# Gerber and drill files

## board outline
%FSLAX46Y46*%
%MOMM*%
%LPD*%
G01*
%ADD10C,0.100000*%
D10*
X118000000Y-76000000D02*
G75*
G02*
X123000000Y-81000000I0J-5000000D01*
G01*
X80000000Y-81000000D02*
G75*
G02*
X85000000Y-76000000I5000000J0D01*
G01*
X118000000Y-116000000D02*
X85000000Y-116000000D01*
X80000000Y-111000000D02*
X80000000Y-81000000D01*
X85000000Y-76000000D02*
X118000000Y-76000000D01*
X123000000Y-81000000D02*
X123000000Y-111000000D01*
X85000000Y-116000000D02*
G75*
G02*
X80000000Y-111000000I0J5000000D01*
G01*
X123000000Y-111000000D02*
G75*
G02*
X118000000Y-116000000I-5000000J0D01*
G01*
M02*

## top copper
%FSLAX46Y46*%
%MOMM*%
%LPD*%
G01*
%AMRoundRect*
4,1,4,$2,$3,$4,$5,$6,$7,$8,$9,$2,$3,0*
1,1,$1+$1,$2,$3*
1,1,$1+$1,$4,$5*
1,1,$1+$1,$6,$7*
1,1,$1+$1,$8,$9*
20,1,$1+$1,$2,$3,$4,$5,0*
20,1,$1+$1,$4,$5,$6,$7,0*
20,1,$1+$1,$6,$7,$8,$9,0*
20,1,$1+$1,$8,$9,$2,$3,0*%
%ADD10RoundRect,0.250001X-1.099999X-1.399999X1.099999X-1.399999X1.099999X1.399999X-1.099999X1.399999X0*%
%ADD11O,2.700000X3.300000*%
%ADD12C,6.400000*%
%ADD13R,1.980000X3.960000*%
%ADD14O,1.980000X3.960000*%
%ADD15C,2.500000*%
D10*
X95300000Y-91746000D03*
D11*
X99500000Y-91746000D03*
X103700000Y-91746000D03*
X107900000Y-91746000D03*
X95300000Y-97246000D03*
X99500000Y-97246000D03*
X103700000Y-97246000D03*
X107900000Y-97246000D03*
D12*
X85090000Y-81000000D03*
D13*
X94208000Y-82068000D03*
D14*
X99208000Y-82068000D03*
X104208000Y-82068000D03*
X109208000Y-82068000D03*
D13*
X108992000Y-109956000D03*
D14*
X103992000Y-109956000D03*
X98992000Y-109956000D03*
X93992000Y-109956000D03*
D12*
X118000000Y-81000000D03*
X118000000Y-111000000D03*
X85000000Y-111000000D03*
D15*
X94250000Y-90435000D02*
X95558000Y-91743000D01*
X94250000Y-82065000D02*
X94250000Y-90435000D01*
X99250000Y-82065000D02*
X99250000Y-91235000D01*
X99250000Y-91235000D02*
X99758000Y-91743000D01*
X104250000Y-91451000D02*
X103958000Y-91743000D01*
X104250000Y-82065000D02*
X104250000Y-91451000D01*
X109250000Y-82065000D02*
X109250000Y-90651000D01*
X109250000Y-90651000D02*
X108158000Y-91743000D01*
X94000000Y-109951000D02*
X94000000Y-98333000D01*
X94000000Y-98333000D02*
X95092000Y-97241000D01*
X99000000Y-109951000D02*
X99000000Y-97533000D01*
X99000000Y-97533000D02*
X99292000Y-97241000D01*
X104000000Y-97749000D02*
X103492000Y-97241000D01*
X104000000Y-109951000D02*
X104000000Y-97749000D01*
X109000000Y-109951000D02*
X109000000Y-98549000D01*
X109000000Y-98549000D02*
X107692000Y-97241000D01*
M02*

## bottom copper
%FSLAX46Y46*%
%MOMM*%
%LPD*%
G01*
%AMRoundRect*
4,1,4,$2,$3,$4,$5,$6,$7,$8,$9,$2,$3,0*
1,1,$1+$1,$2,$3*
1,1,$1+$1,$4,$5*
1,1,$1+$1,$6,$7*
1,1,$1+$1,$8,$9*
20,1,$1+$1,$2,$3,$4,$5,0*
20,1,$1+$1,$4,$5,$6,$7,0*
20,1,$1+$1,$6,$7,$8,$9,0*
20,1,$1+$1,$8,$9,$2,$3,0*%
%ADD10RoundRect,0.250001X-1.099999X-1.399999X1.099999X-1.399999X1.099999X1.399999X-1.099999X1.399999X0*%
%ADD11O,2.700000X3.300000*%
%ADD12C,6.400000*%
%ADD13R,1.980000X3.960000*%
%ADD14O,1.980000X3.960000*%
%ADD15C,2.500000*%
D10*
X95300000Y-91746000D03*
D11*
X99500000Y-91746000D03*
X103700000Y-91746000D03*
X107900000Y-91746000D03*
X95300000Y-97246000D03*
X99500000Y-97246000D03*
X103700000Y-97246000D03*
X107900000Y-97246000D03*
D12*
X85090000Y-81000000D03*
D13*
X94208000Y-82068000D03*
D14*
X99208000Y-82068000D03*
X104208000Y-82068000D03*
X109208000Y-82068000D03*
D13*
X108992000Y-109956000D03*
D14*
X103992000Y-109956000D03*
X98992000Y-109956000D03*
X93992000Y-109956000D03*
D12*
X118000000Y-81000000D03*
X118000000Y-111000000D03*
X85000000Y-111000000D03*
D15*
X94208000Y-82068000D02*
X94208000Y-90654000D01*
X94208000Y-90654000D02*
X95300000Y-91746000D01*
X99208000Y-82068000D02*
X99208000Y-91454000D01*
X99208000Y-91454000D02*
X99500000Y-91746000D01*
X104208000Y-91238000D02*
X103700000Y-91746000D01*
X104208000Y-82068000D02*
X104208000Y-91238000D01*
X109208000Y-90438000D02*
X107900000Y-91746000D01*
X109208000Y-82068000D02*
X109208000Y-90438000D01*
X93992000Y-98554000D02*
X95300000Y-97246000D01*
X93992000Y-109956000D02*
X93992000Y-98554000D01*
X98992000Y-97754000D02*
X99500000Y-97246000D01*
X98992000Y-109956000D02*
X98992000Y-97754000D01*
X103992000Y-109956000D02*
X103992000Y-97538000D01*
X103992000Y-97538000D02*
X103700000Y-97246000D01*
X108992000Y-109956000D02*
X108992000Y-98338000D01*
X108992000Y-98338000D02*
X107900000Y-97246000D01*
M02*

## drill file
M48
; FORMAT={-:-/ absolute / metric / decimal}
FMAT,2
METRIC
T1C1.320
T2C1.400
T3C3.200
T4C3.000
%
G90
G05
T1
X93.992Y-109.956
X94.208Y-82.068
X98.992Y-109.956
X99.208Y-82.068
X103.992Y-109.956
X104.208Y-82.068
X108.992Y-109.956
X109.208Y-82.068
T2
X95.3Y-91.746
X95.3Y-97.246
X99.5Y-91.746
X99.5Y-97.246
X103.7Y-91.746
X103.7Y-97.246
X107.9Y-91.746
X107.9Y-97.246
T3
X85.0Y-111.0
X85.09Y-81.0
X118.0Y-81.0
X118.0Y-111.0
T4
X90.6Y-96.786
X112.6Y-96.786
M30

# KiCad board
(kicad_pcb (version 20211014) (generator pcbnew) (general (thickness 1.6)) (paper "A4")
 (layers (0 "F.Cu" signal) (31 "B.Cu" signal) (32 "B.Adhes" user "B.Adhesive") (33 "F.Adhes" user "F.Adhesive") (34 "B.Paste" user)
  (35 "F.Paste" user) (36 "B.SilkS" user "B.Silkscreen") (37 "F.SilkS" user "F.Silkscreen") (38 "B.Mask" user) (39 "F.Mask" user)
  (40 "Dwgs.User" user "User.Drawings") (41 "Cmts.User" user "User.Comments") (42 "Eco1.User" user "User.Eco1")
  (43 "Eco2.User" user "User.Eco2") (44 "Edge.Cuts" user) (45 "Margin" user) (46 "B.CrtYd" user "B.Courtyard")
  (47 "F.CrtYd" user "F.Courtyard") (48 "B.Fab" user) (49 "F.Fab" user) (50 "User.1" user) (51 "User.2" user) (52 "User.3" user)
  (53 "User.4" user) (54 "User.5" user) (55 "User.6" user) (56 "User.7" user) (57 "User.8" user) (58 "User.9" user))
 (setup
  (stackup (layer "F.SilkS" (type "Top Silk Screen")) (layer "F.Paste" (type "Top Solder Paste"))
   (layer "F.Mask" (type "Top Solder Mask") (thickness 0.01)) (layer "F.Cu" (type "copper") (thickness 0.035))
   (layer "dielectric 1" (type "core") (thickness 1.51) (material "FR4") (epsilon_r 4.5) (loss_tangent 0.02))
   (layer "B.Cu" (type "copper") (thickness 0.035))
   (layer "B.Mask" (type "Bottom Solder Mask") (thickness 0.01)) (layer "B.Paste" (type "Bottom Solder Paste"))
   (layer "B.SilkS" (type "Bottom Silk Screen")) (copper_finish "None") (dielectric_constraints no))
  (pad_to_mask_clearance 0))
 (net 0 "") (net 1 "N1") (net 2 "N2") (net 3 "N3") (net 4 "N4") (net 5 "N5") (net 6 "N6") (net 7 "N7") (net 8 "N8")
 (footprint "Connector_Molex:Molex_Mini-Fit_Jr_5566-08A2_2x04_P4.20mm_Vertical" (layer "F.Cu") (at 95.3 91.746)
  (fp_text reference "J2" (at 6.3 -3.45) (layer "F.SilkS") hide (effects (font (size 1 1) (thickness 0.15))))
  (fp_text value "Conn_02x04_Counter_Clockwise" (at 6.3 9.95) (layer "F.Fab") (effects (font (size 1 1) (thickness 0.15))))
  (pad "" np_thru_hole circle (at 17.3 5.04) (size 3 3) (drill 3) (layers *.Cu *.Mask))
  (pad "" np_thru_hole circle (at -4.7 5.04) (size 3 3) (drill 3) (layers *.Cu *.Mask))
  (pad "1" thru_hole roundrect (at 0 0) (size 2.7 3.3) (drill 1.4) (layers *.Cu *.Mask) (roundrect_rratio 0.092593) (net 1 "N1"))
  (pad "2" thru_hole oval (at 4.2 0) (size 2.7 3.3) (drill 1.4) (layers *.Cu *.Mask) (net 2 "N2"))
  (pad "3" thru_hole oval (at 8.4 0) (size 2.7 3.3) (drill 1.4) (layers *.Cu *.Mask) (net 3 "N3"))
  (pad "4" thru_hole oval (at 12.6 0) (size 2.7 3.3) (drill 1.4) (layers *.Cu *.Mask) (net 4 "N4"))
  (pad "5" thru_hole oval (at 0 5.5) (size 2.7 3.3) (drill 1.4) (layers *.Cu *.Mask) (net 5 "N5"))
  (pad "6" thru_hole oval (at 4.2 5.5) (size 2.7 3.3) (drill 1.4) (layers *.Cu *.Mask) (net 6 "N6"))
  (pad "7" thru_hole oval (at 8.4 5.5) (size 2.7 3.3) (drill 1.4) (layers *.Cu *.Mask) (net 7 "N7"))
  (pad "8" thru_hole oval (at 12.6 5.5) (size 2.7 3.3) (drill 1.4) (layers *.Cu *.Mask) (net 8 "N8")))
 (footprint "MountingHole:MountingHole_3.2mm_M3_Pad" (layer "F.Cu") (at 85.09 81)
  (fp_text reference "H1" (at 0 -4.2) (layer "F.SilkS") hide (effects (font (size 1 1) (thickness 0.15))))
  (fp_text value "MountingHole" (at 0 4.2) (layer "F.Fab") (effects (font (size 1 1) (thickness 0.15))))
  (pad "1" thru_hole circle (at 0 0) (size 6.4 6.4) (drill 3.2) (layers *.Cu *.Mask)))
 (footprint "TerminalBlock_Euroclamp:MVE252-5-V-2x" (layer "F.Cu") (at 101.6 82.296)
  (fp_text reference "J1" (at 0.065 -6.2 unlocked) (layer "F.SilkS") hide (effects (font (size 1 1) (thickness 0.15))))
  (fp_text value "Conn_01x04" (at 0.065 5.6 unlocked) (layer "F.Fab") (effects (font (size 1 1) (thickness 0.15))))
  (pad "1" thru_hole rect (at -7.392 -0.228) (size 1.98 3.96) (drill 1.32) (layers *.Cu *.Mask) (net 1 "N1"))
  (pad "2" thru_hole oval (at -2.392 -0.228) (size 1.98 3.96) (drill 1.32) (layers *.Cu *.Mask) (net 2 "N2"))
  (pad "3" thru_hole oval (at 2.608 -0.228) (size 1.98 3.96) (drill 1.32) (layers *.Cu *.Mask) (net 3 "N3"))
  (pad "4" thru_hole oval (at 7.608 -0.228) (size 1.98 3.96) (drill 1.32) (layers *.Cu *.Mask) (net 4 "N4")))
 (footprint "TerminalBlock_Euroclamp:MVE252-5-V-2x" (layer "F.Cu") (at 101.6 109.728 180)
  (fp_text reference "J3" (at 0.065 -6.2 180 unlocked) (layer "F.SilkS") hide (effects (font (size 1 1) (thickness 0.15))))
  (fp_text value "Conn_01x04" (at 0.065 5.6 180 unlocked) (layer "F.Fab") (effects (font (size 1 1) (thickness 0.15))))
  (pad "1" thru_hole rect (at -7.392 -0.228 180) (size 1.98 3.96) (drill 1.32) (layers *.Cu *.Mask) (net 8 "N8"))
  (pad "2" thru_hole oval (at -2.392 -0.228 180) (size 1.98 3.96) (drill 1.32) (layers *.Cu *.Mask) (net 7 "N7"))
  (pad "3" thru_hole oval (at 2.608 -0.228 180) (size 1.98 3.96) (drill 1.32) (layers *.Cu *.Mask) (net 6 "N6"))
  (pad "4" thru_hole oval (at 7.608 -0.228 180) (size 1.98 3.96) (drill 1.32) (layers *.Cu *.Mask) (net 5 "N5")))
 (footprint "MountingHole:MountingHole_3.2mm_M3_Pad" (layer "F.Cu") (at 118 81)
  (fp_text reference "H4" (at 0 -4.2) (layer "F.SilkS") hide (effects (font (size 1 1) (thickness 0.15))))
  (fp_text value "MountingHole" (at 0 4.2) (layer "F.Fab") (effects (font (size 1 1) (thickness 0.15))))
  (pad "1" thru_hole circle (at 0 0) (size 6.4 6.4) (drill 3.2) (layers *.Cu *.Mask)))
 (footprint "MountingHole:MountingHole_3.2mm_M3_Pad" (layer "F.Cu") (at 118 111)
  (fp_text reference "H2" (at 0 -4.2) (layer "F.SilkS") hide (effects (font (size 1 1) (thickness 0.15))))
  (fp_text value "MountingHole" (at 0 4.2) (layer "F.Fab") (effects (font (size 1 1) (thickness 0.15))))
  (pad "1" thru_hole circle (at 0 0) (size 6.4 6.4) (drill 3.2) (layers *.Cu *.Mask)))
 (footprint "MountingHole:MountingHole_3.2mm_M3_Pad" (layer "F.Cu") (at 85 111)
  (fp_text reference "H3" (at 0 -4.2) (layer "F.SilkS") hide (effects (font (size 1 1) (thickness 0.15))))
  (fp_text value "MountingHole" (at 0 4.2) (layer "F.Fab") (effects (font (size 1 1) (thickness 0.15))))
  (pad "1" thru_hole circle (at 0 0) (size 6.4 6.4) (drill 3.2) (layers *.Cu *.Mask)))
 (gr_arc (start 118 76) (mid 121.535534 77.464466) (end 123 81) (layer "Edge.Cuts") (width 0.1))
 (gr_arc (start 80 81) (mid 81.464466 77.464466) (end 85 76) (layer "Edge.Cuts") (width 0.1))
 (gr_line (start 118 116) (end 85 116) (layer "Edge.Cuts") (width 0.1))
 (gr_line (start 80 111) (end 80 81) (layer "Edge.Cuts") (width 0.1))
 (gr_line (start 85 76) (end 118 76) (layer "Edge.Cuts") (width 0.1))
 (gr_line (start 123 81) (end 123 111) (layer "Edge.Cuts") (width 0.1))
 (gr_arc (start 85 116) (mid 81.464466 114.535534) (end 80 111) (layer "Edge.Cuts") (width 0.1))
 (gr_arc (start 123 111) (mid 121.535534 114.535534) (end 118 116) (layer "Edge.Cuts") (width 0.1))
 (segment (start 94.25 90.435) (end 95.558 91.743) (width 2.5) (layer "F.Cu") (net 1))
 (segment (start 94.25 82.065) (end 94.25 90.435) (width 2.5) (layer "F.Cu") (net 1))
 (segment (start 94.208 82.068) (end 94.208 90.654) (width 2.5) (layer "B.Cu") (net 1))
 (segment (start 94.208 90.654) (end 95.3 91.746) (width 2.5) (layer "B.Cu") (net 1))
 (segment (start 99.25 82.065) (end 99.25 91.235) (width 2.5) (layer "F.Cu") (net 2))
 (segment (start 99.25 91.235) (end 99.758 91.743) (width 2.5) (layer "F.Cu") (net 2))
 (segment (start 99.208 82.068) (end 99.208 91.454) (width 2.5) (layer "B.Cu") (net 2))
 (segment (start 99.208 91.454) (end 99.5 91.746) (width 2.5) (layer "B.Cu") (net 2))
 (segment (start 104.25 91.451) (end 103.958 91.743) (width 2.5) (layer "F.Cu") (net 3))
 (segment (start 104.25 82.065) (end 104.25 91.451) (width 2.5) (layer "F.Cu") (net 3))
 (segment (start 104.208 91.238) (end 103.7 91.746) (width 2.5) (layer "B.Cu") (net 3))
 (segment (start 104.208 82.068) (end 104.208 91.238) (width 2.5) (layer "B.Cu") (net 3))
 (segment (start 109.25 82.065) (end 109.25 90.651) (width 2.5) (layer "F.Cu") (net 4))
 (segment (start 109.25 90.651) (end 108.158 91.743) (width 2.5) (layer "F.Cu") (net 4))
 (segment (start 109.208 90.438) (end 107.9 91.746) (width 2.5) (layer "B.Cu") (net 4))
 (segment (start 109.208 82.068) (end 109.208 90.438) (width 2.5) (layer "B.Cu") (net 4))
 (segment (start 94 109.951) (end 94 98.333) (width 2.5) (layer "F.Cu") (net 5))
 (segment (start 94 98.333) (end 95.092 97.241) (width 2.5) (layer "F.Cu") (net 5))
 (segment (start 93.992 98.554) (end 95.3 97.246) (width 2.5) (layer "B.Cu") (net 5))
 (segment (start 93.992 109.956) (end 93.992 98.554) (width 2.5) (layer "B.Cu") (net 5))
 (segment (start 99 109.951) (end 99 97.533) (width 2.5) (layer "F.Cu") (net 6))
 (segment (start 99 97.533) (end 99.292 97.241) (width 2.5) (layer "F.Cu") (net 6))
 (segment (start 98.992 97.754) (end 99.5 97.246) (width 2.5) (layer "B.Cu") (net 6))
 (segment (start 98.992 109.956) (end 98.992 97.754) (width 2.5) (layer "B.Cu") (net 6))
 (segment (start 104 97.749) (end 103.492 97.241) (width 2.5) (layer "F.Cu") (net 7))
 (segment (start 104 109.951) (end 104 97.749) (width 2.5) (layer "F.Cu") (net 7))
 (segment (start 103.992 109.956) (end 103.992 97.538) (width 2.5) (layer "B.Cu") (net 7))
 (segment (start 103.992 97.538) (end 103.7 97.246) (width 2.5) (layer "B.Cu") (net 7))
 (segment (start 109 109.951) (end 109 98.549) (width 2.5) (layer "F.Cu") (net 8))
 (segment (start 109 98.549) (end 107.692 97.241) (width 2.5) (layer "F.Cu") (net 8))
 (segment (start 108.992 109.956) (end 108.992 98.338) (width 2.5) (layer "B.Cu") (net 8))
 (segment (start 108.992 98.338) (end 107.9 97.246) (width 2.5) (layer "B.Cu") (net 8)))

